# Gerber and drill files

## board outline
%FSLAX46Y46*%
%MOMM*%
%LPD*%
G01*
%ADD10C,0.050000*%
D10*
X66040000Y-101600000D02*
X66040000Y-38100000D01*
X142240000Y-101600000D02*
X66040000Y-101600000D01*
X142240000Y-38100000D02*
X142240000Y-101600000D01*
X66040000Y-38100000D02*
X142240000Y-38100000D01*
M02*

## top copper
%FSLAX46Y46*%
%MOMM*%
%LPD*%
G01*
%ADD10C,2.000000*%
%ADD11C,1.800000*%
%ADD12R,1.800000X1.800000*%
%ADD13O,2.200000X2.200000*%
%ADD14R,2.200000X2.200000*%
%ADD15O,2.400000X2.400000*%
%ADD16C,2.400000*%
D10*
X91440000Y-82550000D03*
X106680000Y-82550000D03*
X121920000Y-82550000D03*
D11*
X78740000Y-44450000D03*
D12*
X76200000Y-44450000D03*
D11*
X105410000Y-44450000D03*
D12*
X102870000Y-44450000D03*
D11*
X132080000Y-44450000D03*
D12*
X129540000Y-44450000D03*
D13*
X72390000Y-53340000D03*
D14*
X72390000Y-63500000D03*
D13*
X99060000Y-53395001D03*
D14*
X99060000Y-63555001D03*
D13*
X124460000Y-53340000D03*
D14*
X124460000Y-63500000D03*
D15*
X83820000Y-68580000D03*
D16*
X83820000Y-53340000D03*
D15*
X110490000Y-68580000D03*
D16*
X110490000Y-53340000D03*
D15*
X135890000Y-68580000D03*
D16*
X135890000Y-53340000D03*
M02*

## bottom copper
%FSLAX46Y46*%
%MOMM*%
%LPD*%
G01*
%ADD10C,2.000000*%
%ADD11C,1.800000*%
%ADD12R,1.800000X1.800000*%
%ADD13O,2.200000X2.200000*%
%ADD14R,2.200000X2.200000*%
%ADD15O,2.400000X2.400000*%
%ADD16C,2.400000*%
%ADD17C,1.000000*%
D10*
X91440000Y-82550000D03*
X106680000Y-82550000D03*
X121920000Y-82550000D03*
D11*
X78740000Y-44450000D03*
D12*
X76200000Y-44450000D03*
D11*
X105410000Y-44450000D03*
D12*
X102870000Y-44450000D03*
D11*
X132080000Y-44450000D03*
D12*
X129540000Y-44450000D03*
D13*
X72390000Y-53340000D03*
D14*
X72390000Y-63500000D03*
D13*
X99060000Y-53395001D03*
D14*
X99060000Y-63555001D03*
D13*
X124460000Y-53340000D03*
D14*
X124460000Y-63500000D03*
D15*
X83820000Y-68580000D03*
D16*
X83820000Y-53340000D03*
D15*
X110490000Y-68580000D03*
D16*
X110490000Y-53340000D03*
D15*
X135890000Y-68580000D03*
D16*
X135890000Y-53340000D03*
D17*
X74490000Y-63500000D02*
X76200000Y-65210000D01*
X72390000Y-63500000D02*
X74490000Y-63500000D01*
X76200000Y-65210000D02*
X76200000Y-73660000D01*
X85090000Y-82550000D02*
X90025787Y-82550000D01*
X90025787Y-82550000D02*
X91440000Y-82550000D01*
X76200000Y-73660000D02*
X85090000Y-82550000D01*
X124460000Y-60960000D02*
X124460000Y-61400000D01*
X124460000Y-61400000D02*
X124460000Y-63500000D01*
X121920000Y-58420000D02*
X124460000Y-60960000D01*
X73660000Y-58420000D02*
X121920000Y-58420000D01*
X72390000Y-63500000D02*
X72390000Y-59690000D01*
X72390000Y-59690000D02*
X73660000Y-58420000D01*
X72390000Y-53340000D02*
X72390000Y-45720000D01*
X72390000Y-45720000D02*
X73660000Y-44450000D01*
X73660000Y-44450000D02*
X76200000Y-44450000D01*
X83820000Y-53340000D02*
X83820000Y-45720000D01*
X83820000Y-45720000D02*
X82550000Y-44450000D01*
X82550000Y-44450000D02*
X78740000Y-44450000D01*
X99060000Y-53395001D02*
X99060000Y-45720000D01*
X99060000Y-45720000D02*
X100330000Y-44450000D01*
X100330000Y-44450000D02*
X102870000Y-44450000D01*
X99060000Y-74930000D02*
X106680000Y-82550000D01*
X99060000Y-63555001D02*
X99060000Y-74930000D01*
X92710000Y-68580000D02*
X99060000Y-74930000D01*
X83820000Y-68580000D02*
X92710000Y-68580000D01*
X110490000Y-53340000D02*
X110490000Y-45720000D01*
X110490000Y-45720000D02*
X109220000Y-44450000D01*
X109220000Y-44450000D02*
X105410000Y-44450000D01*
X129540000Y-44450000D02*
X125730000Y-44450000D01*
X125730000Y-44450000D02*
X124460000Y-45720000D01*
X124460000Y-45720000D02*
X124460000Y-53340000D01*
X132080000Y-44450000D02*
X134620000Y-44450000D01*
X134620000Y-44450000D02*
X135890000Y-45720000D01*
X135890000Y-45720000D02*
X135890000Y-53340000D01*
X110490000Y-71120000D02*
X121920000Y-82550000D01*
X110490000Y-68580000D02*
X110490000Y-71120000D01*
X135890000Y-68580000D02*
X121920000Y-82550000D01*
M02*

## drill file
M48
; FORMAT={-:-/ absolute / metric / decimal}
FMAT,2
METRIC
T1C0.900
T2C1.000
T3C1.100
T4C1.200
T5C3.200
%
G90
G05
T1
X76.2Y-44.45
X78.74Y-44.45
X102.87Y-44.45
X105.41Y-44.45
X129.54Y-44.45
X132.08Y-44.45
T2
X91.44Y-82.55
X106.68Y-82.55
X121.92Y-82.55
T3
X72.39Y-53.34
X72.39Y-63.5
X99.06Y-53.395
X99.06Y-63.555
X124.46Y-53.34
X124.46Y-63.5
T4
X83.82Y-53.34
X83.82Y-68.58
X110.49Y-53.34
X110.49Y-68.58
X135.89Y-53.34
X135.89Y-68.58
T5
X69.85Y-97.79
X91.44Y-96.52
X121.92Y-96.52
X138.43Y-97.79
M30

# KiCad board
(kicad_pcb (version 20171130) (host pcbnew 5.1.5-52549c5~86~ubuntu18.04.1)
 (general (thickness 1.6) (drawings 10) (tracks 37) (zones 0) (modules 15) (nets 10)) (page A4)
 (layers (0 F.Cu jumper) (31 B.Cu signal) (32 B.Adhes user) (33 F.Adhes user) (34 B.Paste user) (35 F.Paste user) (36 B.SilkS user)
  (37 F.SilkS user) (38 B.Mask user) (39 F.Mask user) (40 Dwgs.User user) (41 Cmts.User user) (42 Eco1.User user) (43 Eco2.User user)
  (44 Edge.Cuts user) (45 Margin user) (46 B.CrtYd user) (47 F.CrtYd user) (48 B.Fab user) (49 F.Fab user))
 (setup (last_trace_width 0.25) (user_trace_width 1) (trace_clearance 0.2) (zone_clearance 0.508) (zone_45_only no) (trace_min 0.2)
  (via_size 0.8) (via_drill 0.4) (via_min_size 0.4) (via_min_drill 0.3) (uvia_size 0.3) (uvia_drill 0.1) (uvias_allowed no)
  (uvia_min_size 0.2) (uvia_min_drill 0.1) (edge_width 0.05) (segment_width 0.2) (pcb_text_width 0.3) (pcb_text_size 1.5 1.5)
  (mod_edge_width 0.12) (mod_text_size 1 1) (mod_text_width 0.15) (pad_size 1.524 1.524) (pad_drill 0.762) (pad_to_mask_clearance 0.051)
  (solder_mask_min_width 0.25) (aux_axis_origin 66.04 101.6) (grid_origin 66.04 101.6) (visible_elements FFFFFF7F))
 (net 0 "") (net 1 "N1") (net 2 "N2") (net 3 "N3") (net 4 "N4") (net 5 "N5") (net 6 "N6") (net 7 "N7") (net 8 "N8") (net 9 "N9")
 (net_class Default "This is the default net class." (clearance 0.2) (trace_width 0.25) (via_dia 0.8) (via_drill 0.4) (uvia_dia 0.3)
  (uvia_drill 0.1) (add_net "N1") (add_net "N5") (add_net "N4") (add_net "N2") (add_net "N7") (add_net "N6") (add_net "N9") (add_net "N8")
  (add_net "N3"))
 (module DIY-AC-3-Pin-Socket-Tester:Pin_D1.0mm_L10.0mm (layer F.Cu) (at 91.44 82.55)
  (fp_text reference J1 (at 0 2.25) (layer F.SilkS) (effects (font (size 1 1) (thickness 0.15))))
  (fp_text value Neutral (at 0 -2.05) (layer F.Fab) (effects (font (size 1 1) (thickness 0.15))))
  (pad 1 thru_hole circle (at 0 0) (size 2 2) (drill 1) (layers *.Cu *.Mask) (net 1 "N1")))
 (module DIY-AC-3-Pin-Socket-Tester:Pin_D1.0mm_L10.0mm (layer F.Cu) (at 106.68 82.55)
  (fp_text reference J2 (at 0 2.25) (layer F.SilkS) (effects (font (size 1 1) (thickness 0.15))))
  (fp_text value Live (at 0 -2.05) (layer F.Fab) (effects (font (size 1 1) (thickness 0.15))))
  (pad 1 thru_hole circle (at 0 0) (size 2 2) (drill 1) (layers *.Cu *.Mask) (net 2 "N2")))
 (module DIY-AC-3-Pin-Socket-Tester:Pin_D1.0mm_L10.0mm (layer F.Cu) (at 121.92 82.55)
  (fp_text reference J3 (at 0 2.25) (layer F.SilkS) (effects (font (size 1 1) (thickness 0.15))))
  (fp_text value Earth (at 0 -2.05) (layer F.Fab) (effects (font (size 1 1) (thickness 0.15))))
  (pad 1 thru_hole circle (at 0 0) (size 2 2) (drill 1) (layers *.Cu *.Mask) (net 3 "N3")))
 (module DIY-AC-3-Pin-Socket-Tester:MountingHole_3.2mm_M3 (layer F.Cu) (at 138.43 97.79)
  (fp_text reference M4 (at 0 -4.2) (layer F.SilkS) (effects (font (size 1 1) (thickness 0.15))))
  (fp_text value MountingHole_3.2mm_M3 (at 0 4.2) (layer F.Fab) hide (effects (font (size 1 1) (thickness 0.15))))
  (pad 1 np_thru_hole circle (at 0 0) (size 3.2 3.2) (drill 3.2) (layers *.Cu *.Mask)))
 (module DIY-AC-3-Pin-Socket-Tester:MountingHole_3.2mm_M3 (layer F.Cu) (at 69.85 97.79)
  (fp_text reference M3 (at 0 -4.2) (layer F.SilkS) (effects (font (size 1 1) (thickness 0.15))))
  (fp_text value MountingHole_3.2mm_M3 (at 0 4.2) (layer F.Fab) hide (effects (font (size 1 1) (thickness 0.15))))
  (pad 1 np_thru_hole circle (at 0 0) (size 3.2 3.2) (drill 3.2) (layers *.Cu *.Mask)))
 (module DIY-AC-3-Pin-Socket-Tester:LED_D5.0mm (layer F.Cu) (at 76.2 44.45)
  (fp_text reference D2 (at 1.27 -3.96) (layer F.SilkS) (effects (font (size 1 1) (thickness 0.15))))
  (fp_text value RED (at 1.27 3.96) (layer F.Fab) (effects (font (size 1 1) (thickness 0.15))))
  (pad 2 thru_hole circle (at 2.54 0) (size 1.8 1.8) (drill 0.9) (layers *.Cu *.Mask) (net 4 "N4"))
  (pad 1 thru_hole rect (at 0 0) (size 1.8 1.8) (drill 0.9) (layers *.Cu *.Mask) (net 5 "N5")))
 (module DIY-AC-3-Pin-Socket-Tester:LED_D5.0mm (layer F.Cu) (at 102.87 44.45)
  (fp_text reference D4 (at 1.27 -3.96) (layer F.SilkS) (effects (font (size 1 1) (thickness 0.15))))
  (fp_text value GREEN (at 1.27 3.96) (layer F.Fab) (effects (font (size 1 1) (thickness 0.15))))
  (pad 2 thru_hole circle (at 2.54 0) (size 1.8 1.8) (drill 0.9) (layers *.Cu *.Mask) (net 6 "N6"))
  (pad 1 thru_hole rect (at 0 0) (size 1.8 1.8) (drill 0.9) (layers *.Cu *.Mask) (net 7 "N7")))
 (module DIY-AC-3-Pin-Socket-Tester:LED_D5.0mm (layer F.Cu) (at 129.54 44.45)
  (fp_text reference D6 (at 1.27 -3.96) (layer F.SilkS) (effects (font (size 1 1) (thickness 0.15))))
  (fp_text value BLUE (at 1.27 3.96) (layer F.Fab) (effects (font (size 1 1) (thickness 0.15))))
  (pad 2 thru_hole circle (at 2.54 0) (size 1.8 1.8) (drill 0.9) (layers *.Cu *.Mask) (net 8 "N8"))
  (pad 1 thru_hole rect (at 0 0) (size 1.8 1.8) (drill 0.9) (layers *.Cu *.Mask) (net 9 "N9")))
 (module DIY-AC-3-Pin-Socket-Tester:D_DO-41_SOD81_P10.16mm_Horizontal (layer F.Cu) (at 72.39 63.5 90)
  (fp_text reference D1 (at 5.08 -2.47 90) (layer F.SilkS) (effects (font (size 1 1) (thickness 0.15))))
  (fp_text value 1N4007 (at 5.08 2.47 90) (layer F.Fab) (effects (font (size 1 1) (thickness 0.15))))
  (pad 2 thru_hole oval (at 10.16 0 90) (size 2.2 2.2) (drill 1.1) (layers *.Cu *.Mask) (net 5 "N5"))
  (pad 1 thru_hole rect (at 0 0 90) (size 2.2 2.2) (drill 1.1) (layers *.Cu *.Mask) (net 1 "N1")))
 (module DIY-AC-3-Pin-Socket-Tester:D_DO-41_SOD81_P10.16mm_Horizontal (layer F.Cu) (at 99.06 63.555001 90)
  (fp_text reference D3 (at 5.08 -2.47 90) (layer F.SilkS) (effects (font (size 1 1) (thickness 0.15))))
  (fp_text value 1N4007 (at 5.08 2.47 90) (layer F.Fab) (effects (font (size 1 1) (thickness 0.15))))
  (pad 2 thru_hole oval (at 10.16 0 90) (size 2.2 2.2) (drill 1.1) (layers *.Cu *.Mask) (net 7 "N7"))
  (pad 1 thru_hole rect (at 0 0 90) (size 2.2 2.2) (drill 1.1) (layers *.Cu *.Mask) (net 2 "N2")))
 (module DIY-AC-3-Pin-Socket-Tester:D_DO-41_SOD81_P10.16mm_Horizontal (layer F.Cu) (at 124.46 63.5 90)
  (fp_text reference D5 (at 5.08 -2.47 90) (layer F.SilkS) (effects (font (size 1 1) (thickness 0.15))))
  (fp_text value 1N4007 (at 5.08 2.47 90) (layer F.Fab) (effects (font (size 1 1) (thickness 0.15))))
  (pad 2 thru_hole oval (at 10.16 0 90) (size 2.2 2.2) (drill 1.1) (layers *.Cu *.Mask) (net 9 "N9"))
  (pad 1 thru_hole rect (at 0 0 90) (size 2.2 2.2) (drill 1.1) (layers *.Cu *.Mask) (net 1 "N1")))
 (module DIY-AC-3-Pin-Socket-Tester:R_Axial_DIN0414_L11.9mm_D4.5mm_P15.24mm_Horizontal (layer F.Cu) (at 83.82 53.34 270)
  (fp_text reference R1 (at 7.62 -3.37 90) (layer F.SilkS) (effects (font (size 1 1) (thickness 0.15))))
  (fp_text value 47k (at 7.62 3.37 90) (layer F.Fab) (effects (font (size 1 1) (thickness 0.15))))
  (pad 2 thru_hole oval (at 15.24 0 270) (size 2.4 2.4) (drill 1.2) (layers *.Cu *.Mask) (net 2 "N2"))
  (pad 1 thru_hole circle (at 0 0 270) (size 2.4 2.4) (drill 1.2) (layers *.Cu *.Mask) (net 4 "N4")))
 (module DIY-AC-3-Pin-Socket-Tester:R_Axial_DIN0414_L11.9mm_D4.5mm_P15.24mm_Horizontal (layer F.Cu) (at 110.49 53.34 270)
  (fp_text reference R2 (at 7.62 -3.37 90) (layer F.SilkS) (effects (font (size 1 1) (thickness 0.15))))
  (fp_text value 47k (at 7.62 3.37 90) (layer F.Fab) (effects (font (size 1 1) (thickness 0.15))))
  (pad 2 thru_hole oval (at 15.24 0 270) (size 2.4 2.4) (drill 1.2) (layers *.Cu *.Mask) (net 3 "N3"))
  (pad 1 thru_hole circle (at 0 0 270) (size 2.4 2.4) (drill 1.2) (layers *.Cu *.Mask) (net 6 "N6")))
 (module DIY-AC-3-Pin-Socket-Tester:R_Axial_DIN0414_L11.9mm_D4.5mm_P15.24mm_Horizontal (layer F.Cu) (at 135.89 53.34 270)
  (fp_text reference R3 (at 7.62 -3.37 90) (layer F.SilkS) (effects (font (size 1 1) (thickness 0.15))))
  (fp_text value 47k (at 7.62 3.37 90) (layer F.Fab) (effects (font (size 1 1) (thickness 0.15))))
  (pad 2 thru_hole oval (at 15.24 0 270) (size 2.4 2.4) (drill 1.2) (layers *.Cu *.Mask) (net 3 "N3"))
  (pad 1 thru_hole circle (at 0 0 270) (size 2.4 2.4) (drill 1.2) (layers *.Cu *.Mask) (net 8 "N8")))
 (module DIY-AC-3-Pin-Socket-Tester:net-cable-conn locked (layer F.Cu) (at 106.68 96.52)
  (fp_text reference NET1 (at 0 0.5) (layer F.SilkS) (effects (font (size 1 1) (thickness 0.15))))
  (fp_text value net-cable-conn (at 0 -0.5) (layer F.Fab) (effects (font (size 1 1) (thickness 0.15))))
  (pad "" np_thru_hole circle (at 15.24 0) (size 3.2 3.2) (drill 3.2) (layers *.Cu *.Mask))
  (pad "" np_thru_hole circle (at -15.24 0) (size 3.2 3.2) (drill 3.2) (layers *.Cu *.Mask)))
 (gr_line (start 66.04 101.6) (end 66.04 38.1) (layer Edge.Cuts) (width 0.05))
 (gr_line (start 142.24 101.6) (end 66.04 101.6) (layer Edge.Cuts) (width 0.05))
 (gr_line (start 142.24 38.1) (end 142.24 101.6) (layer Edge.Cuts) (width 0.05))
 (gr_line (start 66.04 38.1) (end 142.24 38.1) (layer Edge.Cuts) (width 0.05))
 (segment (start 74.49 63.5) (end 76.2 65.21) (width 1) (layer B.Cu) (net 1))
 (segment (start 72.39 63.5) (end 74.49 63.5) (width 1) (layer B.Cu) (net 1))
 (segment (start 76.2 65.21) (end 76.2 73.66) (width 1) (layer B.Cu) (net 1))
 (segment (start 85.09 82.55) (end 90.025787 82.55) (width 1) (layer B.Cu) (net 1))
 (segment (start 90.025787 82.55) (end 91.44 82.55) (width 1) (layer B.Cu) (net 1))
 (segment (start 76.2 73.66) (end 85.09 82.55) (width 1) (layer B.Cu) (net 1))
 (segment (start 124.46 60.96) (end 124.46 61.4) (width 1) (layer B.Cu) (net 1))
 (segment (start 124.46 61.4) (end 124.46 63.5) (width 1) (layer B.Cu) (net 1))
 (segment (start 121.92 58.42) (end 124.46 60.96) (width 1) (layer B.Cu) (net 1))
 (segment (start 73.66 58.42) (end 121.92 58.42) (width 1) (layer B.Cu) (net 1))
 (segment (start 72.39 63.5) (end 72.39 59.69) (width 1) (layer B.Cu) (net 1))
 (segment (start 72.39 59.69) (end 73.66 58.42) (width 1) (layer B.Cu) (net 1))
 (segment (start 72.39 53.34) (end 72.39 45.72) (width 1) (layer B.Cu) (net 5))
 (segment (start 72.39 45.72) (end 73.66 44.45) (width 1) (layer B.Cu) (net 5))
 (segment (start 73.66 44.45) (end 76.2 44.45) (width 1) (layer B.Cu) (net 5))
 (segment (start 83.82 53.34) (end 83.82 45.72) (width 1) (layer B.Cu) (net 4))
 (segment (start 83.82 45.72) (end 82.55 44.45) (width 1) (layer B.Cu) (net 4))
 (segment (start 82.55 44.45) (end 78.74 44.45) (width 1) (layer B.Cu) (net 4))
 (segment (start 99.06 53.395001) (end 99.06 45.72) (width 1) (layer B.Cu) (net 7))
 (segment (start 99.06 45.72) (end 100.33 44.45) (width 1) (layer B.Cu) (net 7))
 (segment (start 100.33 44.45) (end 102.87 44.45) (width 1) (layer B.Cu) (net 7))
 (segment (start 99.06 74.93) (end 106.68 82.55) (width 1) (layer B.Cu) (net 2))
 (segment (start 99.06 63.555001) (end 99.06 74.93) (width 1) (layer B.Cu) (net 2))
 (segment (start 92.71 68.58) (end 99.06 74.93) (width 1) (layer B.Cu) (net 2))
 (segment (start 83.82 68.58) (end 92.71 68.58) (width 1) (layer B.Cu) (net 2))
 (segment (start 110.49 53.34) (end 110.49 45.72) (width 1) (layer B.Cu) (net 6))
 (segment (start 110.49 45.72) (end 109.22 44.45) (width 1) (layer B.Cu) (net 6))
 (segment (start 109.22 44.45) (end 105.41 44.45) (width 1) (layer B.Cu) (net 6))
 (segment (start 129.54 44.45) (end 125.73 44.45) (width 1) (layer B.Cu) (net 9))
 (segment (start 125.73 44.45) (end 124.46 45.72) (width 1) (layer B.Cu) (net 9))
 (segment (start 124.46 45.72) (end 124.46 53.34) (width 1) (layer B.Cu) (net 9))
 (segment (start 132.08 44.45) (end 134.62 44.45) (width 1) (layer B.Cu) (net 8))
 (segment (start 134.62 44.45) (end 135.89 45.72) (width 1) (layer B.Cu) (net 8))
 (segment (start 135.89 45.72) (end 135.89 53.34) (width 1) (layer B.Cu) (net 8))
 (segment (start 110.49 71.12) (end 121.92 82.55) (width 1) (layer B.Cu) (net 3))
 (segment (start 110.49 68.58) (end 110.49 71.12) (width 1) (layer B.Cu) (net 3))
 (segment (start 135.89 68.58) (end 121.92 82.55) (width 1) (layer B.Cu) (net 3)))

